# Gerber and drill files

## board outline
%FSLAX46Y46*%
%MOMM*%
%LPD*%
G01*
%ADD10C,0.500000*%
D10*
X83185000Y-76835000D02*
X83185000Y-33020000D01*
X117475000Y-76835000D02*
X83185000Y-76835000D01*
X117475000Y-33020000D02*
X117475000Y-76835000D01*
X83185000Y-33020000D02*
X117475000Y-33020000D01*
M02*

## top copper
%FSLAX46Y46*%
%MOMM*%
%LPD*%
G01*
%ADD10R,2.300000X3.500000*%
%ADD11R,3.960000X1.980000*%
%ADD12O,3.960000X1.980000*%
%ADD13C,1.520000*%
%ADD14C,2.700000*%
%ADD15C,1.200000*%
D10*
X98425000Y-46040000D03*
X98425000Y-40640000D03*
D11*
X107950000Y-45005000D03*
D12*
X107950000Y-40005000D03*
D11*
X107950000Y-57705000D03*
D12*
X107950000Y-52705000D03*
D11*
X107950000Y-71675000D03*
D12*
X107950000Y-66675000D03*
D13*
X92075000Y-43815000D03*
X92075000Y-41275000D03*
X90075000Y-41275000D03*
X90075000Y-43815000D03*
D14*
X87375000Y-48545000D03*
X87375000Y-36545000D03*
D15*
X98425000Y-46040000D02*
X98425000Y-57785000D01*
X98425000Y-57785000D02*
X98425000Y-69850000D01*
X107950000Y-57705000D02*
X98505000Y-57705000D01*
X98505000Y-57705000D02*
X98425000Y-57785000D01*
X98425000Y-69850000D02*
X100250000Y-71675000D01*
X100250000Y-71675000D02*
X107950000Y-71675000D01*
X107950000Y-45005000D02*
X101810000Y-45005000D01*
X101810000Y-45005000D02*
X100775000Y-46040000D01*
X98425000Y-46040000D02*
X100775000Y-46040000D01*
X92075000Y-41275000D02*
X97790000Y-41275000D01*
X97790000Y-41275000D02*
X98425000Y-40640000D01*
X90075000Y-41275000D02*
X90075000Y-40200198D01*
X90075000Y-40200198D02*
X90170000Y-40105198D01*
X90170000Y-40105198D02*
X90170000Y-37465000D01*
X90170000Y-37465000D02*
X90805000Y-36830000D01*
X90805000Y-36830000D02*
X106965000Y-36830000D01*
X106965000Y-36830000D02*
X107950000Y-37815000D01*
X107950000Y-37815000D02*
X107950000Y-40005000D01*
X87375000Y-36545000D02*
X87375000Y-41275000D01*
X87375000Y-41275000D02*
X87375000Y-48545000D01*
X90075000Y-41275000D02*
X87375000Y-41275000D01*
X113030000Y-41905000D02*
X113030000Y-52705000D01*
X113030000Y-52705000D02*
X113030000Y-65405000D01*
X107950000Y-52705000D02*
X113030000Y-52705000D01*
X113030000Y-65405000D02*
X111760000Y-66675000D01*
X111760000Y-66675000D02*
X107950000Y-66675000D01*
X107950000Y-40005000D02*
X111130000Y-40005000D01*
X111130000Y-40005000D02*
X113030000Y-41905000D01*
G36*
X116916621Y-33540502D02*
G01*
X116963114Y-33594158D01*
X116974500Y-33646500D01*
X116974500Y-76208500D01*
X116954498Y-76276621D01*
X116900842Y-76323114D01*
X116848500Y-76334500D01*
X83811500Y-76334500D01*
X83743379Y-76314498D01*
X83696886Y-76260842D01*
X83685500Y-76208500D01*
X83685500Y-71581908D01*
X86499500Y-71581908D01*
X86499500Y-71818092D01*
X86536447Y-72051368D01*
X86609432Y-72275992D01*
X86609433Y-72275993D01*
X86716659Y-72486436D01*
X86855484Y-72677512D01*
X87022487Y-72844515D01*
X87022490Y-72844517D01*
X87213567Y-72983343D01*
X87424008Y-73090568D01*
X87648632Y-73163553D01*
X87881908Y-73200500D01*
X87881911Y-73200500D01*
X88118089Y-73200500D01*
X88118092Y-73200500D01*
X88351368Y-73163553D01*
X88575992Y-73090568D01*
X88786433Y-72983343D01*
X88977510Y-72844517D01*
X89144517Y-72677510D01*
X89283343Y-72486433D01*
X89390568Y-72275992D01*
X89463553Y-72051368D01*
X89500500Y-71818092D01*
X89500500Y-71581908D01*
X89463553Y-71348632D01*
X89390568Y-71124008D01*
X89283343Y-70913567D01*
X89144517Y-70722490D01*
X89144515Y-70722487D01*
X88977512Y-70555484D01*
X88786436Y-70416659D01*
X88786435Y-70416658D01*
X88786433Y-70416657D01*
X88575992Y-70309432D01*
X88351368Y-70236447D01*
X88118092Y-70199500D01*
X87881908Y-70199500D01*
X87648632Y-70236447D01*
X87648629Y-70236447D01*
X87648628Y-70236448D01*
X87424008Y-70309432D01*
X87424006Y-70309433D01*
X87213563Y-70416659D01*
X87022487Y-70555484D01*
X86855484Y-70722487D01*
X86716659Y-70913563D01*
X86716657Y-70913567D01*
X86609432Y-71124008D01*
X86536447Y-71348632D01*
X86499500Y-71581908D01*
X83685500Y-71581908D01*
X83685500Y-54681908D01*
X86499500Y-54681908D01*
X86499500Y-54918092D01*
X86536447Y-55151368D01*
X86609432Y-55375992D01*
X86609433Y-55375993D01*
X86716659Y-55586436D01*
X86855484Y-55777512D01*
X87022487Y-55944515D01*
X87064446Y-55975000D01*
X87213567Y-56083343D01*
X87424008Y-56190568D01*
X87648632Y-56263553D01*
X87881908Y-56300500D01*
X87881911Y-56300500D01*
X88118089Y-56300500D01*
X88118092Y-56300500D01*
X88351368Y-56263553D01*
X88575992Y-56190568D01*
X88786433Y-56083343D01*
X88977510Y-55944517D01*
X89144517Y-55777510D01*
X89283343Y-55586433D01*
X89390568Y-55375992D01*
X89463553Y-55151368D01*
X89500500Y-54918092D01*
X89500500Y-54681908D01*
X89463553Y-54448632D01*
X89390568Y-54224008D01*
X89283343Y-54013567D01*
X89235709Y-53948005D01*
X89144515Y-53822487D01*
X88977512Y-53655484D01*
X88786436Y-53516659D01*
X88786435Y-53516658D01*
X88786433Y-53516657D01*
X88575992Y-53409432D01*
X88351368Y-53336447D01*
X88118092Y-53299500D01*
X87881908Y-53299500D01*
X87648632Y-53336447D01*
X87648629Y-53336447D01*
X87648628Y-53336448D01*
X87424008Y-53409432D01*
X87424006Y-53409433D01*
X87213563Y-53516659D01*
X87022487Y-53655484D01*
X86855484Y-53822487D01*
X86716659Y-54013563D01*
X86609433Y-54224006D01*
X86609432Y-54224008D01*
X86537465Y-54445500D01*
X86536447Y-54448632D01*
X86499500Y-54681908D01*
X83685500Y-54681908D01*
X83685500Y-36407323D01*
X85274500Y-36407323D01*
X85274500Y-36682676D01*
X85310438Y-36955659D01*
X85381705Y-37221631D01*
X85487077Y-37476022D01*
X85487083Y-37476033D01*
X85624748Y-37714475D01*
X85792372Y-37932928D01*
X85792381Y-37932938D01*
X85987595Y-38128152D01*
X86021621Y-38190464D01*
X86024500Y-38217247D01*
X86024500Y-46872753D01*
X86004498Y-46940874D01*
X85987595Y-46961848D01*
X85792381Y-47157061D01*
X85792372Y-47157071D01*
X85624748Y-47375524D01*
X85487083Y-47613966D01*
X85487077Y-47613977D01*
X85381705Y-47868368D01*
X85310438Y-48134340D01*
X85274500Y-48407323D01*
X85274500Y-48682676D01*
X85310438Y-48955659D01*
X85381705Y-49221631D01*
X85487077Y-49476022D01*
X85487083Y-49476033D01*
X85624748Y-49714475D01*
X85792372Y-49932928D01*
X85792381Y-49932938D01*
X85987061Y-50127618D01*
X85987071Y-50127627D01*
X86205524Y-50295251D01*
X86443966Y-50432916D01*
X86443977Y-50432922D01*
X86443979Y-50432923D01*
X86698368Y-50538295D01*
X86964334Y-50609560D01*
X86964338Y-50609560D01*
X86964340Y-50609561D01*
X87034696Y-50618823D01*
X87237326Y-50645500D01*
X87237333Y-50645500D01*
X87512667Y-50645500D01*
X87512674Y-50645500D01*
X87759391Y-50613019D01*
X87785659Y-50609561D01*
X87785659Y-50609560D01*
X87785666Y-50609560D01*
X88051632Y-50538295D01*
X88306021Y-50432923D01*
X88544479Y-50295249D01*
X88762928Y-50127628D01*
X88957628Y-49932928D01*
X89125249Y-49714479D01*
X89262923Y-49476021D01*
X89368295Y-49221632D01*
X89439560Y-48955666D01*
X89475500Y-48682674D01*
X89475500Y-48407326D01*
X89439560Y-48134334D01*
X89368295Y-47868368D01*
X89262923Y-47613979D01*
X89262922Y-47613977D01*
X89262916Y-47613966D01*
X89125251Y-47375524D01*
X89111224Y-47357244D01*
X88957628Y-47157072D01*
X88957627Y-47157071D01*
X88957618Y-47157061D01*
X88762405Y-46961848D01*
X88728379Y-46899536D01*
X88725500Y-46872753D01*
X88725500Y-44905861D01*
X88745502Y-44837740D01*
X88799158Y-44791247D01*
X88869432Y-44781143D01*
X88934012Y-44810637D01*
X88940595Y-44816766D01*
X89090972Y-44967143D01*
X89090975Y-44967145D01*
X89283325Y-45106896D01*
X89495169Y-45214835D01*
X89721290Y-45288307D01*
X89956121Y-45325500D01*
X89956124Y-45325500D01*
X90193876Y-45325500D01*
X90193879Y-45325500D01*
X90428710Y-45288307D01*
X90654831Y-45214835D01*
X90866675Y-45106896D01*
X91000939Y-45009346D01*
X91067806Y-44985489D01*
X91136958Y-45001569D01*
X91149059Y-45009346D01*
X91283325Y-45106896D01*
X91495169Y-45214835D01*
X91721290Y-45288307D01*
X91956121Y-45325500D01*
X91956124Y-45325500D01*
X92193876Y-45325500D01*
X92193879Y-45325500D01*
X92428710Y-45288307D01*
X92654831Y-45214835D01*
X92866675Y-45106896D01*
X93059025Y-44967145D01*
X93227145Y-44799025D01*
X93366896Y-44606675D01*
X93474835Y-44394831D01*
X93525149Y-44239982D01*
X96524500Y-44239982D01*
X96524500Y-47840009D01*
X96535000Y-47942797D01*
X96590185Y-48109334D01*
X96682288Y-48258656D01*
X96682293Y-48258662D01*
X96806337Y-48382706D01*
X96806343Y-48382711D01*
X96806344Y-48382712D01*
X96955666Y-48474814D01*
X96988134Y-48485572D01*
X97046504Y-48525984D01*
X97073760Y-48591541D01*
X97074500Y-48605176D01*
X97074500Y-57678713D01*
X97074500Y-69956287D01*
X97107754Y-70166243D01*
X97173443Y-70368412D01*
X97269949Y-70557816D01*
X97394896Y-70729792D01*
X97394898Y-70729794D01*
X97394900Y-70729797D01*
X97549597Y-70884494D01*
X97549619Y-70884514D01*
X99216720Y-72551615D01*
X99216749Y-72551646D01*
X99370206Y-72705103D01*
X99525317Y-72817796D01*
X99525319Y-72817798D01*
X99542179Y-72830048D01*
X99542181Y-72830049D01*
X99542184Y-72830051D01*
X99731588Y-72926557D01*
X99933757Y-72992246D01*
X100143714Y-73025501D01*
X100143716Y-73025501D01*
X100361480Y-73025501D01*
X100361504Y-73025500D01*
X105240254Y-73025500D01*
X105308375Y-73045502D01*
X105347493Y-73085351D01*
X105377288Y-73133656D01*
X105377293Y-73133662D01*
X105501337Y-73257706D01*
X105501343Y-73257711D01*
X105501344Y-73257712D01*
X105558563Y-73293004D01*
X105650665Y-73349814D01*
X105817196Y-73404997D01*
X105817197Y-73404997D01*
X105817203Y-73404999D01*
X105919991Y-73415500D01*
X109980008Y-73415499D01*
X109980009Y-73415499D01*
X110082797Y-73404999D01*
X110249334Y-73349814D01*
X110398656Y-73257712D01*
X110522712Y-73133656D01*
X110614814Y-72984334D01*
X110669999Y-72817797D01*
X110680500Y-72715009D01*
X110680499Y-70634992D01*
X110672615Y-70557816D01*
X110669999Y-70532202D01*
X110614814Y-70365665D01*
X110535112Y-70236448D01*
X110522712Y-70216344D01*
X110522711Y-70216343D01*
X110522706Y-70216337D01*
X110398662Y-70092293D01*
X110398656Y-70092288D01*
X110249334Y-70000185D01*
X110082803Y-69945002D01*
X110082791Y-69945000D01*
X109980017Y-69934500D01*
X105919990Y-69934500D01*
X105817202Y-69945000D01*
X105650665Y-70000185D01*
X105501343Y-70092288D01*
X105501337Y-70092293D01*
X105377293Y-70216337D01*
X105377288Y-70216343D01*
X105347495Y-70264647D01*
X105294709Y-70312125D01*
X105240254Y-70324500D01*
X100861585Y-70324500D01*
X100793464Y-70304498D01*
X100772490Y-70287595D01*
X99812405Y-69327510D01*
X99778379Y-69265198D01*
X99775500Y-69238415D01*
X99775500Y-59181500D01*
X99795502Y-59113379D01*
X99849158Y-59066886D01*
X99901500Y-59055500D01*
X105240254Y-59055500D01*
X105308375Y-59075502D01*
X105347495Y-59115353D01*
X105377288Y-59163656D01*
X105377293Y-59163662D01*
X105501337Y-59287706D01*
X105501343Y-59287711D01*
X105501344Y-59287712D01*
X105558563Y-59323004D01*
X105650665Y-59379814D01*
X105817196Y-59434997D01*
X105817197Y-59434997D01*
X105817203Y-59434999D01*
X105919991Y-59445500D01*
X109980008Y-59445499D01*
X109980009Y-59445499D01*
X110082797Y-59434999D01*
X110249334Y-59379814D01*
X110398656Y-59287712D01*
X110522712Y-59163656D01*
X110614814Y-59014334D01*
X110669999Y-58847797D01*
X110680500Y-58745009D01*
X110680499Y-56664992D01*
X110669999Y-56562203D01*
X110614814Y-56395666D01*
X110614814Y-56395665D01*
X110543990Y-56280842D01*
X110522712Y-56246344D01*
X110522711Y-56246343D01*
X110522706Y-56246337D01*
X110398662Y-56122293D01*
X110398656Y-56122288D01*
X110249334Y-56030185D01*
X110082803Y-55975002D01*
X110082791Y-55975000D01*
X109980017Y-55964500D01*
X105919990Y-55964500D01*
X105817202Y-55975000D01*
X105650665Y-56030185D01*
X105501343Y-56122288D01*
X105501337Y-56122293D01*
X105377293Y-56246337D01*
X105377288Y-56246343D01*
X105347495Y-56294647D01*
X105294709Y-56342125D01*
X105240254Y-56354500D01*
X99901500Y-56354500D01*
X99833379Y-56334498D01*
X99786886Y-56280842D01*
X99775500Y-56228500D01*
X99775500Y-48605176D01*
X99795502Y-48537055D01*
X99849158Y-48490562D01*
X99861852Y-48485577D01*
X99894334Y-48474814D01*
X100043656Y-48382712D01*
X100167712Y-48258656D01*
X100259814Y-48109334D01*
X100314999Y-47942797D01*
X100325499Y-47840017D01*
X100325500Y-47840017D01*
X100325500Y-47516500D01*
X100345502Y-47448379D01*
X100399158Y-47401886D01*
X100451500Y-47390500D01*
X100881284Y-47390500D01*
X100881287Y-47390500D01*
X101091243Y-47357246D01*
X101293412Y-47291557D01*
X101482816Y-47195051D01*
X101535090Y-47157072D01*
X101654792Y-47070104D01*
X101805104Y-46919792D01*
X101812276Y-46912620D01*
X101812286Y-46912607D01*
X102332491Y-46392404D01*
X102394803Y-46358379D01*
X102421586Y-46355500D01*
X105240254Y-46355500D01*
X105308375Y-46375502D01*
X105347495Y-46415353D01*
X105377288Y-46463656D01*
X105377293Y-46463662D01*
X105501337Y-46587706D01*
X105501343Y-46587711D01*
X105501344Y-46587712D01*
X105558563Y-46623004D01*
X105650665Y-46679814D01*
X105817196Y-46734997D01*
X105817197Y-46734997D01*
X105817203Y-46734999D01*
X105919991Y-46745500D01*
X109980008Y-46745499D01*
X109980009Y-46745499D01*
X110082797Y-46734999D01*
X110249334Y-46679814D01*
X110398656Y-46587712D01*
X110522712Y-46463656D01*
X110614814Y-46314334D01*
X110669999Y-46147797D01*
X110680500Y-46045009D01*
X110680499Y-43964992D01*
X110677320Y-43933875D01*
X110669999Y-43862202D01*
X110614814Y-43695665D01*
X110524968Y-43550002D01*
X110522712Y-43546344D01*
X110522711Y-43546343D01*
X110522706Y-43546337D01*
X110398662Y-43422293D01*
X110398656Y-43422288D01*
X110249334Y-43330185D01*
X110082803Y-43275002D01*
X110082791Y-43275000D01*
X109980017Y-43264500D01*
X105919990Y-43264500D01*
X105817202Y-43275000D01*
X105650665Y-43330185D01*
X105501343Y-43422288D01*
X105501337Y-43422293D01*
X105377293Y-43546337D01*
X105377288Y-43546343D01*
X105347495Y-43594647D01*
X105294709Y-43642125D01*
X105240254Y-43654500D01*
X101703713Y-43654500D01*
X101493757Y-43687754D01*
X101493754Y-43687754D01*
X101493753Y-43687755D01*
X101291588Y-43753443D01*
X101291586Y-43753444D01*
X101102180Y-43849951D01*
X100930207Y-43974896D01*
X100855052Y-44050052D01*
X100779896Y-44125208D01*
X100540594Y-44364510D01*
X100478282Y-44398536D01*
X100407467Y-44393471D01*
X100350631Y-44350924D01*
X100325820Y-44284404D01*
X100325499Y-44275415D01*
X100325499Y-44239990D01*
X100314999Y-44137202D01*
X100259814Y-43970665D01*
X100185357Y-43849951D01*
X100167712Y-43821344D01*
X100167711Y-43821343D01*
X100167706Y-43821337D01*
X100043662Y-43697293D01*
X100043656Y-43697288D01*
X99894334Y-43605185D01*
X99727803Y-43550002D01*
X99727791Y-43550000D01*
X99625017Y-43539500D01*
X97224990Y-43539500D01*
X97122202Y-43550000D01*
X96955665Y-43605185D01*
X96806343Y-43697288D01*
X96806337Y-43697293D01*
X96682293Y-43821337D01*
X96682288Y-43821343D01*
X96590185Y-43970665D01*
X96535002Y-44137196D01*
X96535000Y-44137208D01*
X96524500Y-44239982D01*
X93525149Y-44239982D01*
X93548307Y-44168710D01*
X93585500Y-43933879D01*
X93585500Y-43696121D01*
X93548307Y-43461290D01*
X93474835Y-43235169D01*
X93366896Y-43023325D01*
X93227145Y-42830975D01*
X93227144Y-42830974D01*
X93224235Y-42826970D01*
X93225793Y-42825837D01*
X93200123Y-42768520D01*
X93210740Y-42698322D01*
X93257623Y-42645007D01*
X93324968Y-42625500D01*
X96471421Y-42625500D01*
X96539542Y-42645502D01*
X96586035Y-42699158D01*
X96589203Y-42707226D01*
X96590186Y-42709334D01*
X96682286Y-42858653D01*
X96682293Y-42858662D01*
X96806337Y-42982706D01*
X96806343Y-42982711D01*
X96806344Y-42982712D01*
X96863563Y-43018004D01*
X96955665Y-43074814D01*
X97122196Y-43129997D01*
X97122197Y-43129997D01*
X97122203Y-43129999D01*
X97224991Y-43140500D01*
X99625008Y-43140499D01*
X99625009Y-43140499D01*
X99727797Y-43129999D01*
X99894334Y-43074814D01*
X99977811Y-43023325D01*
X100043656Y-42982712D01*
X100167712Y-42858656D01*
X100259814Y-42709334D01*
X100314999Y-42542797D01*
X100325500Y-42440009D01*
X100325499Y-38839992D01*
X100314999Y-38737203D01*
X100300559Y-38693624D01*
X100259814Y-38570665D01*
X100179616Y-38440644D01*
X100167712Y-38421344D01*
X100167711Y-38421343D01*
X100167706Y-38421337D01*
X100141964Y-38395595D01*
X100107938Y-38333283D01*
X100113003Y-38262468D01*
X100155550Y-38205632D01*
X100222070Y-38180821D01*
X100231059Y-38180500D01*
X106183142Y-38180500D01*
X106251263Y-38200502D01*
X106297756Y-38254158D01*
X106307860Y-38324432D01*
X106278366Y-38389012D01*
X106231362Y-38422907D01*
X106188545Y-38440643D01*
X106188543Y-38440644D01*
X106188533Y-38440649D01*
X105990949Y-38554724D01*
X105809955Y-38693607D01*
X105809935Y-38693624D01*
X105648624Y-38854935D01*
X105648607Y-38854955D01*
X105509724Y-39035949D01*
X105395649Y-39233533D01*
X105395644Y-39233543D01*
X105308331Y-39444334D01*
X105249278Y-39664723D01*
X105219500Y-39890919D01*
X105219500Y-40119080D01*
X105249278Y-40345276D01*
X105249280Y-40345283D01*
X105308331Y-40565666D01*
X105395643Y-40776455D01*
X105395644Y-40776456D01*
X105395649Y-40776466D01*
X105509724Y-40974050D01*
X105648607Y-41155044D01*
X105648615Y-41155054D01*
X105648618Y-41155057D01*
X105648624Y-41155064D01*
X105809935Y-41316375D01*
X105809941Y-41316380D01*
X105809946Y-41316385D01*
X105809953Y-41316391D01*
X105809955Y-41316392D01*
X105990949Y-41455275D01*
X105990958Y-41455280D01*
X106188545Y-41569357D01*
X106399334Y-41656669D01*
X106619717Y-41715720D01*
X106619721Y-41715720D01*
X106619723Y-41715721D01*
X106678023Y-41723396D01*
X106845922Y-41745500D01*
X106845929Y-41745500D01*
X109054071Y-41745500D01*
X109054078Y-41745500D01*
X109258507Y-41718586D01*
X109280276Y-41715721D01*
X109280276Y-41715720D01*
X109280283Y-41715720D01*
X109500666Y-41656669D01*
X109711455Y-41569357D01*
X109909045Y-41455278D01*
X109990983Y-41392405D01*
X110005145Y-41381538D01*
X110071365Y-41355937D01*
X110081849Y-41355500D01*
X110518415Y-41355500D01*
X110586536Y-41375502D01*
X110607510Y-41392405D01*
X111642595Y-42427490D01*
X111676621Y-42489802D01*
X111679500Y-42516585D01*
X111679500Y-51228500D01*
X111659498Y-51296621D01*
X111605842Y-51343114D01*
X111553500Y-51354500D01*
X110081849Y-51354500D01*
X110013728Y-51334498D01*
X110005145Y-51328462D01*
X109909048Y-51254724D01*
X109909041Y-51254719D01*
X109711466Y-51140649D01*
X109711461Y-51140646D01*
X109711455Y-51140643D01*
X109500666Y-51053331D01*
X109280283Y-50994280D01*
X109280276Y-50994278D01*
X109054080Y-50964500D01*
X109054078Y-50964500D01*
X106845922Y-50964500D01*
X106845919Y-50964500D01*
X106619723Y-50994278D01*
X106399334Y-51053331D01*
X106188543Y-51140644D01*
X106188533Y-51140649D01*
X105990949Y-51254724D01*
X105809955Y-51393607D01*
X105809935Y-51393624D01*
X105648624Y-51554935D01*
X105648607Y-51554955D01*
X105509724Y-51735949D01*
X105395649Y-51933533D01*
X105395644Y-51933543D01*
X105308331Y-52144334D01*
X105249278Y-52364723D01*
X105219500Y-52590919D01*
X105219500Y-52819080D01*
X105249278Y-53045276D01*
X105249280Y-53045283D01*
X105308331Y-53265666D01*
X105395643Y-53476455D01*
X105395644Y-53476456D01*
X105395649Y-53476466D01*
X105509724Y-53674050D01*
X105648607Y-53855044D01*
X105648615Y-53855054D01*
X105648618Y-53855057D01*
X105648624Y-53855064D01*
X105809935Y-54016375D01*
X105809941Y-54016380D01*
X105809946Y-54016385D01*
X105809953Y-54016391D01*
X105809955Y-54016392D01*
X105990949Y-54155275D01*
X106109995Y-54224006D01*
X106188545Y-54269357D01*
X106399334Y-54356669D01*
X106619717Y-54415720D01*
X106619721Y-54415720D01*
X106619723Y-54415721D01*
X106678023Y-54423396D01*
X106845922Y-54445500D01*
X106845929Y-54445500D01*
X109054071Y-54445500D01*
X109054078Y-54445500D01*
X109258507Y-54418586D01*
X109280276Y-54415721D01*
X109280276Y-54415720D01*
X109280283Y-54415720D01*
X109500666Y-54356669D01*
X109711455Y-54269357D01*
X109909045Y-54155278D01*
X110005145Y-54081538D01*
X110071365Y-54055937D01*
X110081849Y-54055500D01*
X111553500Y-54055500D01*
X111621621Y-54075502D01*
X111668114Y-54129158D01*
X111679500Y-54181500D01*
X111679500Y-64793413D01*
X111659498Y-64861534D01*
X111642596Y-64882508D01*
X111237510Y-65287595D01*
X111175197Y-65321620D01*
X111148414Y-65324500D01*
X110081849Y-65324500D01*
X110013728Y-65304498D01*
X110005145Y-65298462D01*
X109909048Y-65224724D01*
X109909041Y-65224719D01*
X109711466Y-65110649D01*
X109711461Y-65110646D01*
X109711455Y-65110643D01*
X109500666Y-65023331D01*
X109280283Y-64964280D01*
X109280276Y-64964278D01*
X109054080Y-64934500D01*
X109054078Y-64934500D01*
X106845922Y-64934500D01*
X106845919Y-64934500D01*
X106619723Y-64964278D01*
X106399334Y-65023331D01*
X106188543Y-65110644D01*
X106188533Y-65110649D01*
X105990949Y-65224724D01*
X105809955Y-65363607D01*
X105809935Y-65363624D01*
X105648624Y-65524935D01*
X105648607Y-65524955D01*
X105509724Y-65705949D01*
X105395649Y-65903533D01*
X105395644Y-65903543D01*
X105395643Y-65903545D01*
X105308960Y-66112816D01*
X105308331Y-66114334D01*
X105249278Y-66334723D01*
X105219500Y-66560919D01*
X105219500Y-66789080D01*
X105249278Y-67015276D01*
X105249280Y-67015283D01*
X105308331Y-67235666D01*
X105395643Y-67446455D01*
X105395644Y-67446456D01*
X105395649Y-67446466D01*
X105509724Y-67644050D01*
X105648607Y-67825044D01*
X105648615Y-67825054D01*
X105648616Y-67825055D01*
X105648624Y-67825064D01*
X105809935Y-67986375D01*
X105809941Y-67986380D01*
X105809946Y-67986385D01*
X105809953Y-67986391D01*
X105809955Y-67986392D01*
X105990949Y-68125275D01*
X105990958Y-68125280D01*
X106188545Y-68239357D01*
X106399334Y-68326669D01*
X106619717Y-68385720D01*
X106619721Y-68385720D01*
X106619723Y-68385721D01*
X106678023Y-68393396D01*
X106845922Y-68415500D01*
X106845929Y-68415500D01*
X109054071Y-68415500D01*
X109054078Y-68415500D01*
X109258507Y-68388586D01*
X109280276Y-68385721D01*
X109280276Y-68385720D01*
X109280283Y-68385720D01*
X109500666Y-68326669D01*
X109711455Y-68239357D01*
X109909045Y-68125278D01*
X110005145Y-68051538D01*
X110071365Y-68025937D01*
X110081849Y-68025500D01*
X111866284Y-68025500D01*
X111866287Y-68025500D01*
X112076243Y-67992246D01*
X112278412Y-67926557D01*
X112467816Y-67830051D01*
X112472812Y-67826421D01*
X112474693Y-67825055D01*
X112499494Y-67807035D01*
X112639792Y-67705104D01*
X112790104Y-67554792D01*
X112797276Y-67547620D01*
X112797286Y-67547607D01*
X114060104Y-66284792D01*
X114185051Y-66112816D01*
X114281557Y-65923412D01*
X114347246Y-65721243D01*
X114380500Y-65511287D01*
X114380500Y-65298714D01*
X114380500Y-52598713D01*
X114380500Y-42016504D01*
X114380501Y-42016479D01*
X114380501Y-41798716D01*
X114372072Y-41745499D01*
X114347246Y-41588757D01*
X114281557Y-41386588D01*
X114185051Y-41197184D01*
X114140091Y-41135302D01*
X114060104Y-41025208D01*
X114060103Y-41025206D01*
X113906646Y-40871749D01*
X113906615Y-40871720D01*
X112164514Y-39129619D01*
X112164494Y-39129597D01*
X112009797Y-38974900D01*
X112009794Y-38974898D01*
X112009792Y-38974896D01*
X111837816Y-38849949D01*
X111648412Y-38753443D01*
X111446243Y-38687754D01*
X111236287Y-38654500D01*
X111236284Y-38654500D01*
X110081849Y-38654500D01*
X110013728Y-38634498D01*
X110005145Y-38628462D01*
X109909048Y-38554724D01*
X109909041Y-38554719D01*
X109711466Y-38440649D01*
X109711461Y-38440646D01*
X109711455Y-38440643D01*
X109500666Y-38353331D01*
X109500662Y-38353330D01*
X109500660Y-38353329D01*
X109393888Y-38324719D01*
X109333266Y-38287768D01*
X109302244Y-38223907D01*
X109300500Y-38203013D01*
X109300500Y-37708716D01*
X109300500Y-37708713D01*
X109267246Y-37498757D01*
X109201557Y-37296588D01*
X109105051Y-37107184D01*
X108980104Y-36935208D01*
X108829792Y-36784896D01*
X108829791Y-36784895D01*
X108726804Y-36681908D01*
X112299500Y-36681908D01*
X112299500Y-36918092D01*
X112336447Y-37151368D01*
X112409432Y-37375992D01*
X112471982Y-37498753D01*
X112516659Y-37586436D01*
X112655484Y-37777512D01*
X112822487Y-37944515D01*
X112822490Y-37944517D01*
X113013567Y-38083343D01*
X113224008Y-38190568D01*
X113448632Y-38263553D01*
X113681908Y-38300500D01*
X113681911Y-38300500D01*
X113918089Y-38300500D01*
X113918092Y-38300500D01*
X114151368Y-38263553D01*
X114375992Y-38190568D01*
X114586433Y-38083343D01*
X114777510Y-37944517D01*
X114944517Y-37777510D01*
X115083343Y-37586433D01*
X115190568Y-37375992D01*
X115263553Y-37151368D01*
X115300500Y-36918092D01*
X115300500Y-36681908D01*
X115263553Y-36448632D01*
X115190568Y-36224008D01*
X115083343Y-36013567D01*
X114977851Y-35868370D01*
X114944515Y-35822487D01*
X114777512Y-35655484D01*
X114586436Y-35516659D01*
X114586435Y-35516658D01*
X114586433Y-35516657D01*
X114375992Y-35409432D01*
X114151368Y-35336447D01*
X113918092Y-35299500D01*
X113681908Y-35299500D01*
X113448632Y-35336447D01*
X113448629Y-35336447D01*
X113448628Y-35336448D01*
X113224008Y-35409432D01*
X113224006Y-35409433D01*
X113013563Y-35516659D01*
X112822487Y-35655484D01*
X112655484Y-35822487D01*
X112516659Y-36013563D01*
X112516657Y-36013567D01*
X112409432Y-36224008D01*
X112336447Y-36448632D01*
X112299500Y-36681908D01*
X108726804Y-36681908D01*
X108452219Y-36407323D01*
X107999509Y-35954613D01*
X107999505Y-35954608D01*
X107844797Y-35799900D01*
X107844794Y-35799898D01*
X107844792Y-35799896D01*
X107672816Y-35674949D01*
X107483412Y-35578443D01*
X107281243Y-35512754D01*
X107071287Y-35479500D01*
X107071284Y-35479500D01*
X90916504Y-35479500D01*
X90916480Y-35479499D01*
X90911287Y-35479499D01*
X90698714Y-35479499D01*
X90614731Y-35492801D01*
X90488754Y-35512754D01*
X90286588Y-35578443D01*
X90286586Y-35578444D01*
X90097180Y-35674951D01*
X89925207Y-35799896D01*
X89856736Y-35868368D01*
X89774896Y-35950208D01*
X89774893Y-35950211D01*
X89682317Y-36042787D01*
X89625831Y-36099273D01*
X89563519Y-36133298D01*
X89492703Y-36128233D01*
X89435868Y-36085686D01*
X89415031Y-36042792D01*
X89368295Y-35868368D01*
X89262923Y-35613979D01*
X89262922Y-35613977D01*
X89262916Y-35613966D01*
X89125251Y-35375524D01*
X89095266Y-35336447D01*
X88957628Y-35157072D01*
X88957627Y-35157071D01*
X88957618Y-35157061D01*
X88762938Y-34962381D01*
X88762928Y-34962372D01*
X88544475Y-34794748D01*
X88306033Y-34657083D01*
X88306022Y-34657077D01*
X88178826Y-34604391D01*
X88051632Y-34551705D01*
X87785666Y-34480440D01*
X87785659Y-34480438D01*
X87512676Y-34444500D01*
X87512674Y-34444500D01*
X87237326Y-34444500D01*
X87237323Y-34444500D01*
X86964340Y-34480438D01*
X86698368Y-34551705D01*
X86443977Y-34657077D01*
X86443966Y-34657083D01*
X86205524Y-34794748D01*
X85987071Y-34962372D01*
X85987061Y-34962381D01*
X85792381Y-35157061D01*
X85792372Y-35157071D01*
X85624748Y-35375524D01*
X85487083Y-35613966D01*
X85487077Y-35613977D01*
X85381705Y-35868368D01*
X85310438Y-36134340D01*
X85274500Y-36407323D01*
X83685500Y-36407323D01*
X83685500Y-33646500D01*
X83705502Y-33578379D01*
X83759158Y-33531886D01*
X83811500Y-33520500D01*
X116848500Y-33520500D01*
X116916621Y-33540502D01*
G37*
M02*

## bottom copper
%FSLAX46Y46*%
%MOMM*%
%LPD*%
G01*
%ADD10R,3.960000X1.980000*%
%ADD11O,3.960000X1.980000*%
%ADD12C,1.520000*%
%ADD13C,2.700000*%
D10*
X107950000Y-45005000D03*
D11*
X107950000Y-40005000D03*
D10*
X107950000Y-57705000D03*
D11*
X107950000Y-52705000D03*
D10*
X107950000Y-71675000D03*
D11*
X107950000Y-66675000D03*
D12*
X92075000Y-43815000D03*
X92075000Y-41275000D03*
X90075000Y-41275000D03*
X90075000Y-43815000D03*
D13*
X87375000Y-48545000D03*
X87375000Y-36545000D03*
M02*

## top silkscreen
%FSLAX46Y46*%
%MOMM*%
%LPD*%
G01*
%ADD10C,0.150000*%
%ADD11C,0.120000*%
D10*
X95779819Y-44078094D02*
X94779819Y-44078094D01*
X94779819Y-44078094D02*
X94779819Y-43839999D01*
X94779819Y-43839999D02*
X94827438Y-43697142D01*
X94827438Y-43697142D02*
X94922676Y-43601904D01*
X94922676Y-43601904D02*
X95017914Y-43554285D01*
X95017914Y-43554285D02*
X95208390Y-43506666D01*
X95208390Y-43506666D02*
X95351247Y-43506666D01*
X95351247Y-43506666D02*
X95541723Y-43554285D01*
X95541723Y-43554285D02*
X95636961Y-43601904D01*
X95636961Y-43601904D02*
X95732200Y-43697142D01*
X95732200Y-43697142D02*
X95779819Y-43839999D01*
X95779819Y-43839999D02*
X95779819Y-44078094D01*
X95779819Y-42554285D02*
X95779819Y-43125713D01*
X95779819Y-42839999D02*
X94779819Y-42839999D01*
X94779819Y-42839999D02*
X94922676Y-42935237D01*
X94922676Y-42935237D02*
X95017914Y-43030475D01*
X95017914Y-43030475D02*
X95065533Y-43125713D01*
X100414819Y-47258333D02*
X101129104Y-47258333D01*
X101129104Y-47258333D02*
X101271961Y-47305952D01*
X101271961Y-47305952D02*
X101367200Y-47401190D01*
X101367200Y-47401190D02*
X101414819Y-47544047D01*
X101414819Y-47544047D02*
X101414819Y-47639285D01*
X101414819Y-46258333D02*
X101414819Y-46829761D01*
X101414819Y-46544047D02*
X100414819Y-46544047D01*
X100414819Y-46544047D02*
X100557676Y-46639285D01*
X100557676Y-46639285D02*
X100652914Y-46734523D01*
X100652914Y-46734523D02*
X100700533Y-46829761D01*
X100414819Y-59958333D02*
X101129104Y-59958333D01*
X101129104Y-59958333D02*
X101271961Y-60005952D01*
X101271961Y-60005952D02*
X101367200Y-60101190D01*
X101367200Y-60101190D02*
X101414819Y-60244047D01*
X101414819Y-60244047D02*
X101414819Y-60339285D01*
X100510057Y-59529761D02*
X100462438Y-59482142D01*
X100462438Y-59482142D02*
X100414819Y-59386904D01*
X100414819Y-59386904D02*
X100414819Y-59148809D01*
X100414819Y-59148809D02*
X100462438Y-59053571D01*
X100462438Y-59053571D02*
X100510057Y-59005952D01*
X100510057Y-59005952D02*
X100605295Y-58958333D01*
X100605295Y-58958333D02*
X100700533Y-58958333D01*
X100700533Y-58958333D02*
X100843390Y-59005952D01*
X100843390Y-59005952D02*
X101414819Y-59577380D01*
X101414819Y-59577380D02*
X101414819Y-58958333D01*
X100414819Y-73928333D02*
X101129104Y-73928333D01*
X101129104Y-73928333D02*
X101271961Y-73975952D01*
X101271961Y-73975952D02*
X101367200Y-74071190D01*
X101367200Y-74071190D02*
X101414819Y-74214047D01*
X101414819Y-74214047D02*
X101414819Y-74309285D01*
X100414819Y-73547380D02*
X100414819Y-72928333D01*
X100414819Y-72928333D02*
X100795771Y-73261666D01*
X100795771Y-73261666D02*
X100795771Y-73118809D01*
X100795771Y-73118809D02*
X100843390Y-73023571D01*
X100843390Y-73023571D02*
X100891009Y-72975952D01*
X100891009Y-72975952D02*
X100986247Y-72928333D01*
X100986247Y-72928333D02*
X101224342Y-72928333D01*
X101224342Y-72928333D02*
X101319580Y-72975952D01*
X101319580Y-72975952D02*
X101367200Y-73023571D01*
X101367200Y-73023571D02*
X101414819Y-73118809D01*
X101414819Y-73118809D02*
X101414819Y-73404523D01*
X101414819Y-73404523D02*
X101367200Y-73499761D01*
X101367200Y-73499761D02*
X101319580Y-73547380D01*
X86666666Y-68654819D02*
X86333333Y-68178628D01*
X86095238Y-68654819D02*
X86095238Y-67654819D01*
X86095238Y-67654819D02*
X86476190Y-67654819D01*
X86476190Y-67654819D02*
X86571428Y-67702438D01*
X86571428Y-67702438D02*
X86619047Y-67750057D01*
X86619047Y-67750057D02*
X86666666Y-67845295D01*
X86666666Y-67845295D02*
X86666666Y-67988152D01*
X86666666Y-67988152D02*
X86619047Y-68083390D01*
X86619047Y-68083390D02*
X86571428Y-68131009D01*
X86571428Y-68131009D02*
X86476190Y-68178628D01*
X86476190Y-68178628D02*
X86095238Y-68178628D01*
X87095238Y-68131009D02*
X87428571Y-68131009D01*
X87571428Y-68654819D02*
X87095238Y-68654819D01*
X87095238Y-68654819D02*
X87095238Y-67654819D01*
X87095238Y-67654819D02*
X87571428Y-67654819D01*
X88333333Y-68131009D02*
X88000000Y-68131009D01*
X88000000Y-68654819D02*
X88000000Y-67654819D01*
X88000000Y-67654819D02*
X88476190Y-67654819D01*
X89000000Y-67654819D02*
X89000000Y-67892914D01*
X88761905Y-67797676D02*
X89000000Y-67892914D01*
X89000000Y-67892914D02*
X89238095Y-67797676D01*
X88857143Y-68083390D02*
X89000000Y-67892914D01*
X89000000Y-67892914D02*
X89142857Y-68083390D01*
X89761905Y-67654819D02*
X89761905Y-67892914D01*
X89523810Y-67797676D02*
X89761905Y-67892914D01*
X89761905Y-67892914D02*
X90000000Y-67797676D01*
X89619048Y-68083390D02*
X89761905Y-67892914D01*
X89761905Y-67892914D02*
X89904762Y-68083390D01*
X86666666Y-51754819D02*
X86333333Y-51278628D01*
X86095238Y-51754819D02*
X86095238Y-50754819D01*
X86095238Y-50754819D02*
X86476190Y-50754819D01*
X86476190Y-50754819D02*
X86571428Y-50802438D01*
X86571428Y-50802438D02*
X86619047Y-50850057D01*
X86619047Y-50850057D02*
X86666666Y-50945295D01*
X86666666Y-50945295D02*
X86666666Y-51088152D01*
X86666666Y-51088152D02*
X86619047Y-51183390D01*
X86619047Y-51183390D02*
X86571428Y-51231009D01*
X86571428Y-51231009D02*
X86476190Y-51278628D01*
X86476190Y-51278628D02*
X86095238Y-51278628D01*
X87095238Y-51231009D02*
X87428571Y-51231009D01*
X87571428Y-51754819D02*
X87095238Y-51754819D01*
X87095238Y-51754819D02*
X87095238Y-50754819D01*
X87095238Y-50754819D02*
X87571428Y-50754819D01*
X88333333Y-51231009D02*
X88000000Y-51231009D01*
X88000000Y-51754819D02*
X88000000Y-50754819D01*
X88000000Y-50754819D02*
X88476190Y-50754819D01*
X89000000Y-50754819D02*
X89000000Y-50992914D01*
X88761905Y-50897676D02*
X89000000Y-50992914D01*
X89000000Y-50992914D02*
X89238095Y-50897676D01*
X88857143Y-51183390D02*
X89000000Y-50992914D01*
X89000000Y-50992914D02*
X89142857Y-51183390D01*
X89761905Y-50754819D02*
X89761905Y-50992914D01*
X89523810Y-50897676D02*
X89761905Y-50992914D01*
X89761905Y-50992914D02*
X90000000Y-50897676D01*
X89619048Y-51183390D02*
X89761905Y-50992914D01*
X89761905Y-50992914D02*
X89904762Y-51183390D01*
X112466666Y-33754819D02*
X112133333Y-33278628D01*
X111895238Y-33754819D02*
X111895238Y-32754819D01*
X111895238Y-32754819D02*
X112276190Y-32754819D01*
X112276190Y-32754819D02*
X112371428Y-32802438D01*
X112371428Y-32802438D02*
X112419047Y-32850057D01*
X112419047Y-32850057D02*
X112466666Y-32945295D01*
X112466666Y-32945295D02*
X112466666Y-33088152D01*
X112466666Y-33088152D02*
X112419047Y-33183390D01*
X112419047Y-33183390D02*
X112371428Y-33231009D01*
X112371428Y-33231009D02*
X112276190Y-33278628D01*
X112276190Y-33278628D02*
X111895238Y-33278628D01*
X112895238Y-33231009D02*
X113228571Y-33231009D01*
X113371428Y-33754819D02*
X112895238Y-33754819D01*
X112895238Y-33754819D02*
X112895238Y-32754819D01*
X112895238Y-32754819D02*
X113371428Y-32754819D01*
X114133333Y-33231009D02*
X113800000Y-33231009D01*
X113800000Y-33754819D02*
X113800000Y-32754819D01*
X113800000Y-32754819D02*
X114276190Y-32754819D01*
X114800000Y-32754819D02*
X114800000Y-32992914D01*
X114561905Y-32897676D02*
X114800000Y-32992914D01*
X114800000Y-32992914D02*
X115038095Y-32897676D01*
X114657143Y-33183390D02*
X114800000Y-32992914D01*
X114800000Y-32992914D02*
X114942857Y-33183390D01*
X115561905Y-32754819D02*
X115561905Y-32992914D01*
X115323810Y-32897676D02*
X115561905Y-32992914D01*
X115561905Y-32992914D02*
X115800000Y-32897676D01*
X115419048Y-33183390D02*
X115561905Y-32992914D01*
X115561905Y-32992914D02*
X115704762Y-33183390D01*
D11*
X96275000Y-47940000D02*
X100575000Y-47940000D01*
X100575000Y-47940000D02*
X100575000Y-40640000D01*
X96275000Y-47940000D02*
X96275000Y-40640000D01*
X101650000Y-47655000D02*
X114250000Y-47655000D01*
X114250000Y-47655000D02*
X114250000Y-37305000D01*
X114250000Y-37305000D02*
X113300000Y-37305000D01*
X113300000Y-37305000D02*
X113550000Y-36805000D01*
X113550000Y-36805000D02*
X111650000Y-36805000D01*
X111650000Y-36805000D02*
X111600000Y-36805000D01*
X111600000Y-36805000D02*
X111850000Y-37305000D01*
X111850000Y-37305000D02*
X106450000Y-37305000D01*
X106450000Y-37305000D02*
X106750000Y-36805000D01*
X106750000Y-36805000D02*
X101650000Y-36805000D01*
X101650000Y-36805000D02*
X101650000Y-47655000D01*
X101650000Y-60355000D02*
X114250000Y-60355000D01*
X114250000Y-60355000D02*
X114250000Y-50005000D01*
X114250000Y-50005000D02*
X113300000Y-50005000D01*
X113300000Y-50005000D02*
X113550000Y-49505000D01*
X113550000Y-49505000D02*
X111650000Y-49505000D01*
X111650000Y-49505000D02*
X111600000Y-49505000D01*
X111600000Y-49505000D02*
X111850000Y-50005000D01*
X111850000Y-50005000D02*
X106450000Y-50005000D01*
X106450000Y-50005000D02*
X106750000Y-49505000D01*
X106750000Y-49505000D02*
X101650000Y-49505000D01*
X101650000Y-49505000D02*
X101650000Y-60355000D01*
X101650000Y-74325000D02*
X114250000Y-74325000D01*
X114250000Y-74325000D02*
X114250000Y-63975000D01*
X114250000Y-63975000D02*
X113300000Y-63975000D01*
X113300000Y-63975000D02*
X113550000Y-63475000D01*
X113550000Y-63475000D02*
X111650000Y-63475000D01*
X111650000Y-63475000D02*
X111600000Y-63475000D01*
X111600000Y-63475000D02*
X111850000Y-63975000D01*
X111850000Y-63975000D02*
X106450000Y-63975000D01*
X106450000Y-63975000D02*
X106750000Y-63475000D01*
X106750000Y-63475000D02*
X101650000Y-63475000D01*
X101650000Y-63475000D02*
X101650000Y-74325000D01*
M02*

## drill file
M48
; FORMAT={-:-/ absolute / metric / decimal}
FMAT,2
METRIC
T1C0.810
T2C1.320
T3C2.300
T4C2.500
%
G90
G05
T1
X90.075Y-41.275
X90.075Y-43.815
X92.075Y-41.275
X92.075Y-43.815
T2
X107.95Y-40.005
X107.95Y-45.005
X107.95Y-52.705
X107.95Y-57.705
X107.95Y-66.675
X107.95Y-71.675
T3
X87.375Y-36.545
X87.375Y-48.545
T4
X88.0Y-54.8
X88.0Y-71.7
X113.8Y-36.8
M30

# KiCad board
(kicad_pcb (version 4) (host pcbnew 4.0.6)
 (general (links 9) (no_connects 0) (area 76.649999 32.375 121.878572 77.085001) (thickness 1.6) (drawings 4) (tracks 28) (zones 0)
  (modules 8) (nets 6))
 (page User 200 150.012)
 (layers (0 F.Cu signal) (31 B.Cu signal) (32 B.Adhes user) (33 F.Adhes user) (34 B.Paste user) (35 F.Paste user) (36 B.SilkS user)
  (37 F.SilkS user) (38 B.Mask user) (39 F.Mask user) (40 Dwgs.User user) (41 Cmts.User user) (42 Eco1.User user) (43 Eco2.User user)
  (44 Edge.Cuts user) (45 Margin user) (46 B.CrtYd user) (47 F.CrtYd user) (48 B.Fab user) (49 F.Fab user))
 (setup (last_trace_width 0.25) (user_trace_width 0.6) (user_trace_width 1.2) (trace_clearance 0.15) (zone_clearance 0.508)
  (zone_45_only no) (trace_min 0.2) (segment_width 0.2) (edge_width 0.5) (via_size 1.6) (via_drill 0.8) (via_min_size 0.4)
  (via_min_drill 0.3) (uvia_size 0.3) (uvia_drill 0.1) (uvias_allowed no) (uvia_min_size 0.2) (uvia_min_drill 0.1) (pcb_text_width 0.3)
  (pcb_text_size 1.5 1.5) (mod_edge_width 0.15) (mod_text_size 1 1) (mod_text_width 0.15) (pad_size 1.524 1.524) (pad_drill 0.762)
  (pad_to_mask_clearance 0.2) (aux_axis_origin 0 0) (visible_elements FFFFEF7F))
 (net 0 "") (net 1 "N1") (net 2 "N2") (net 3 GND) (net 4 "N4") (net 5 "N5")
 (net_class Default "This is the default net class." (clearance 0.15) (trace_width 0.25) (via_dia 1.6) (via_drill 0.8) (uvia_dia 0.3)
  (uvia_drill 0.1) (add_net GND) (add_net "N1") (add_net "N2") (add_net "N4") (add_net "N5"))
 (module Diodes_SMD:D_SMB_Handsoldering (layer F.Cu) (at 98.425 43.34 90)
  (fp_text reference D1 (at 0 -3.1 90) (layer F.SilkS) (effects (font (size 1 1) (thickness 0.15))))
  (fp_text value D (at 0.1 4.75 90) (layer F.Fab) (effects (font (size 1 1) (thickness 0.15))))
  (fp_line (start -4.6 -2.15) (end -4.6 2.15) (layer F.SilkS) (width 0.12))
  (fp_line (start -4.6 2.15) (end 2.7 2.15) (layer F.SilkS) (width 0.12))
  (fp_line (start -4.6 -2.15) (end 2.7 -2.15) (layer F.SilkS) (width 0.12))
  (pad 1 smd rect (at -2.7 0 90) (size 3.5 2.3) (layers F.Cu F.Paste F.Mask) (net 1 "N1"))
  (pad 2 smd rect (at 2.7 0 90) (size 3.5 2.3) (layers F.Cu F.Paste F.Mask) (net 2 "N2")))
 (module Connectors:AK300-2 (layer F.Cu) (at 107.95 45.005 90)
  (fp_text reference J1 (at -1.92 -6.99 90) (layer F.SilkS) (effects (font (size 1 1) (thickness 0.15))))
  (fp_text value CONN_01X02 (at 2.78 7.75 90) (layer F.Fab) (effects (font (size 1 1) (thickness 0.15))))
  (fp_line (start -2.65 -6.3) (end -2.65 6.3) (layer F.SilkS) (width 0.12))
  (fp_line (start -2.65 6.3) (end 7.7 6.3) (layer F.SilkS) (width 0.12))
  (fp_line (start 7.7 6.3) (end 7.7 5.35) (layer F.SilkS) (width 0.12))
  (fp_line (start 7.7 5.35) (end 8.2 5.6) (layer F.SilkS) (width 0.12))
  (fp_line (start 8.2 5.6) (end 8.2 3.7) (layer F.SilkS) (width 0.12))
  (fp_line (start 8.2 3.7) (end 8.2 3.65) (layer F.SilkS) (width 0.12))
  (fp_line (start 8.2 3.65) (end 7.7 3.9) (layer F.SilkS) (width 0.12))
  (fp_line (start 7.7 3.9) (end 7.7 -1.5) (layer F.SilkS) (width 0.12))
  (fp_line (start 7.7 -1.5) (end 8.2 -1.2) (layer F.SilkS) (width 0.12))
  (fp_line (start 8.2 -1.2) (end 8.2 -6.3) (layer F.SilkS) (width 0.12))
  (fp_line (start 8.2 -6.3) (end -2.65 -6.3) (layer F.SilkS) (width 0.12))
  (pad 1 thru_hole rect (at 0 0 90) (size 1.98 3.96) (drill 1.32) (layers *.Cu F.Paste F.Mask) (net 1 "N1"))
  (pad 2 thru_hole oval (at 5 0 90) (size 1.98 3.96) (drill 1.32) (layers *.Cu F.Paste F.Mask) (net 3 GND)))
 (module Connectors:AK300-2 (layer F.Cu) (at 107.95 57.705 90)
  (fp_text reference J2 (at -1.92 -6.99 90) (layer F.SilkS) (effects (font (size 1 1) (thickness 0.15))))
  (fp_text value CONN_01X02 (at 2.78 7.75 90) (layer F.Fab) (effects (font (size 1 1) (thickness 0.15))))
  (fp_line (start -2.65 -6.3) (end -2.65 6.3) (layer F.SilkS) (width 0.12))
  (fp_line (start -2.65 6.3) (end 7.7 6.3) (layer F.SilkS) (width 0.12))
  (fp_line (start 7.7 6.3) (end 7.7 5.35) (layer F.SilkS) (width 0.12))
  (fp_line (start 7.7 5.35) (end 8.2 5.6) (layer F.SilkS) (width 0.12))
  (fp_line (start 8.2 5.6) (end 8.2 3.7) (layer F.SilkS) (width 0.12))
  (fp_line (start 8.2 3.7) (end 8.2 3.65) (layer F.SilkS) (width 0.12))
  (fp_line (start 8.2 3.65) (end 7.7 3.9) (layer F.SilkS) (width 0.12))
  (fp_line (start 7.7 3.9) (end 7.7 -1.5) (layer F.SilkS) (width 0.12))
  (fp_line (start 7.7 -1.5) (end 8.2 -1.2) (layer F.SilkS) (width 0.12))
  (fp_line (start 8.2 -1.2) (end 8.2 -6.3) (layer F.SilkS) (width 0.12))
  (fp_line (start 8.2 -6.3) (end -2.65 -6.3) (layer F.SilkS) (width 0.12))
  (pad 1 thru_hole rect (at 0 0 90) (size 1.98 3.96) (drill 1.32) (layers *.Cu F.Paste F.Mask) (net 1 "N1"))
  (pad 2 thru_hole oval (at 5 0 90) (size 1.98 3.96) (drill 1.32) (layers *.Cu F.Paste F.Mask) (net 3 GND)))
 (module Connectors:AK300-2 (layer F.Cu) (at 107.95 71.675 90)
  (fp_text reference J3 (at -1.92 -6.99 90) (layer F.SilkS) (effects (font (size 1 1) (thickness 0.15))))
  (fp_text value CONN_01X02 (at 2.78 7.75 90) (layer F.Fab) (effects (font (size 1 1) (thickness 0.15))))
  (fp_line (start -2.65 -6.3) (end -2.65 6.3) (layer F.SilkS) (width 0.12))
  (fp_line (start -2.65 6.3) (end 7.7 6.3) (layer F.SilkS) (width 0.12))
  (fp_line (start 7.7 6.3) (end 7.7 5.35) (layer F.SilkS) (width 0.12))
  (fp_line (start 7.7 5.35) (end 8.2 5.6) (layer F.SilkS) (width 0.12))
  (fp_line (start 8.2 5.6) (end 8.2 3.7) (layer F.SilkS) (width 0.12))
  (fp_line (start 8.2 3.7) (end 8.2 3.65) (layer F.SilkS) (width 0.12))
  (fp_line (start 8.2 3.65) (end 7.7 3.9) (layer F.SilkS) (width 0.12))
  (fp_line (start 7.7 3.9) (end 7.7 -1.5) (layer F.SilkS) (width 0.12))
  (fp_line (start 7.7 -1.5) (end 8.2 -1.2) (layer F.SilkS) (width 0.12))
  (fp_line (start 8.2 -1.2) (end 8.2 -6.3) (layer F.SilkS) (width 0.12))
  (fp_line (start 8.2 -6.3) (end -2.65 -6.3) (layer F.SilkS) (width 0.12))
  (pad 1 thru_hole rect (at 0 0 90) (size 1.98 3.96) (drill 1.32) (layers *.Cu F.Paste F.Mask) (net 1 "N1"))
  (pad 2 thru_hole oval (at 5 0 90) (size 1.98 3.96) (drill 1.32) (layers *.Cu F.Paste F.Mask) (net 3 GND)))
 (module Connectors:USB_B (layer B.Cu) (at 92.075 41.275 180)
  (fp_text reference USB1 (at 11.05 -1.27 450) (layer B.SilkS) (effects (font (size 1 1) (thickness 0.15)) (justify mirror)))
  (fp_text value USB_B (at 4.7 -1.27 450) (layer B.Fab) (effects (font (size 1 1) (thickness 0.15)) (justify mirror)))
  (pad 2 thru_hole circle (at 0 -2.54 270) (size 1.52 1.52) (drill 0.81) (layers *.Cu *.Mask) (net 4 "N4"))
  (pad 1 thru_hole circle (at 0 0 270) (size 1.52 1.52) (drill 0.81) (layers *.Cu *.Mask) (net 2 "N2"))
  (pad 4 thru_hole circle (at 2 0 270) (size 1.52 1.52) (drill 0.81) (layers *.Cu *.Mask) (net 3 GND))
  (pad 3 thru_hole circle (at 2 -2.54 270) (size 1.52 1.52) (drill 0.81) (layers *.Cu *.Mask) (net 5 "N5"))
  (pad 5 thru_hole circle (at 4.7 -7.27 270) (size 2.7 2.7) (drill 2.3) (layers *.Cu *.Mask) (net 3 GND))
  (pad 5 thru_hole circle (at 4.7 4.73 270) (size 2.7 2.7) (drill 2.3) (layers *.Cu *.Mask) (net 3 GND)))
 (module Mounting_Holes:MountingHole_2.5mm (layer F.Cu) (at 88 71.7)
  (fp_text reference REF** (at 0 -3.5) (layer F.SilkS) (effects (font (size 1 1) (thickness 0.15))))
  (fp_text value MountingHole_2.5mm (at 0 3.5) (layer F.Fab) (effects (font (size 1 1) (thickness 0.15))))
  (pad 1 np_thru_hole circle (at 0 0) (size 2.5 2.5) (drill 2.5) (layers *.Cu *.Mask)))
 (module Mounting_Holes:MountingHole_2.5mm (layer F.Cu) (at 88 54.8)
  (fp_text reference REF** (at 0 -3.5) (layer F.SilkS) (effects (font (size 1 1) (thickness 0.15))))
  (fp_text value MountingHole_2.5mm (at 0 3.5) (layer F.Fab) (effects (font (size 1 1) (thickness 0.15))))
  (pad 1 np_thru_hole circle (at 0 0) (size 2.5 2.5) (drill 2.5) (layers *.Cu *.Mask)))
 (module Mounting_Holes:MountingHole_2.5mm (layer F.Cu) (at 113.8 36.8)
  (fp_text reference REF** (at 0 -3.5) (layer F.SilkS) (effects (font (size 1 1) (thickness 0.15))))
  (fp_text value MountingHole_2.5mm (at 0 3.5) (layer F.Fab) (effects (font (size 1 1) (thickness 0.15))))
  (pad 1 np_thru_hole circle (at 0 0) (size 2.5 2.5) (drill 2.5) (layers *.Cu *.Mask)))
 (gr_line (start 83.185 76.835) (end 83.185 33.02) (layer Edge.Cuts) (width 0.5))
 (gr_line (start 117.475 76.835) (end 83.185 76.835) (layer Edge.Cuts) (width 0.5))
 (gr_line (start 117.475 33.02) (end 117.475 76.835) (layer Edge.Cuts) (width 0.5))
 (gr_line (start 83.185 33.02) (end 117.475 33.02) (layer Edge.Cuts) (width 0.5))
 (segment (start 98.425 46.04) (end 98.425 57.785) (width 1.2) (layer F.Cu) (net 1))
 (segment (start 98.425 57.785) (end 98.425 69.85) (width 1.2) (layer F.Cu) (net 1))
 (segment (start 107.95 57.705) (end 98.505 57.705) (width 1.2) (layer F.Cu) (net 1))
 (segment (start 98.505 57.705) (end 98.425 57.785) (width 1.2) (layer F.Cu) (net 1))
 (segment (start 98.425 69.85) (end 100.25 71.675) (width 1.2) (layer F.Cu) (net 1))
 (segment (start 100.25 71.675) (end 107.95 71.675) (width 1.2) (layer F.Cu) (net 1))
 (segment (start 107.95 45.005) (end 101.81 45.005) (width 1.2) (layer F.Cu) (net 1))
 (segment (start 101.81 45.005) (end 100.775 46.04) (width 1.2) (layer F.Cu) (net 1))
 (segment (start 98.425 46.04) (end 100.775 46.04) (width 1.2) (layer F.Cu) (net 1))
 (segment (start 92.075 41.275) (end 97.79 41.275) (width 1.2) (layer F.Cu) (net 2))
 (segment (start 97.79 41.275) (end 98.425 40.64) (width 1.2) (layer F.Cu) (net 2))
 (segment (start 90.075 41.275) (end 90.075 40.200198) (width 1.2) (layer F.Cu) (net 3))
 (segment (start 90.075 40.200198) (end 90.17 40.105198) (width 1.2) (layer F.Cu) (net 3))
 (segment (start 90.17 40.105198) (end 90.17 37.465) (width 1.2) (layer F.Cu) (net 3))
 (segment (start 90.17 37.465) (end 90.805 36.83) (width 1.2) (layer F.Cu) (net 3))
 (segment (start 90.805 36.83) (end 106.965 36.83) (width 1.2) (layer F.Cu) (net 3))
 (segment (start 106.965 36.83) (end 107.95 37.815) (width 1.2) (layer F.Cu) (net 3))
 (segment (start 107.95 37.815) (end 107.95 40.005) (width 1.2) (layer F.Cu) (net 3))
 (segment (start 87.375 36.545) (end 87.375 41.275) (width 1.2) (layer F.Cu) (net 3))
 (segment (start 87.375 41.275) (end 87.375 48.545) (width 1.2) (layer F.Cu) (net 3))
 (segment (start 90.075 41.275) (end 87.375 41.275) (width 1.2) (layer F.Cu) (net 3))
 (segment (start 113.03 41.905) (end 113.03 52.705) (width 1.2) (layer F.Cu) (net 3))
 (segment (start 113.03 52.705) (end 113.03 65.405) (width 1.2) (layer F.Cu) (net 3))
 (segment (start 107.95 52.705) (end 113.03 52.705) (width 1.2) (layer F.Cu) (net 3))
 (segment (start 113.03 65.405) (end 111.76 66.675) (width 1.2) (layer F.Cu) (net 3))
 (segment (start 111.76 66.675) (end 107.95 66.675) (width 1.2) (layer F.Cu) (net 3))
 (segment (start 107.95 40.005) (end 111.13 40.005) (width 1.2) (layer F.Cu) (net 3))
 (segment (start 111.13 40.005) (end 113.03 41.905) (width 1.2) (layer F.Cu) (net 3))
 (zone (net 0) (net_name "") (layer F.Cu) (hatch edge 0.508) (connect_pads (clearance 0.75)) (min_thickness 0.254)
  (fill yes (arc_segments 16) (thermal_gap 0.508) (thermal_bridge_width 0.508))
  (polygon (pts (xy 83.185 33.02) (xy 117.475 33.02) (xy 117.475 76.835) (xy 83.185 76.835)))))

